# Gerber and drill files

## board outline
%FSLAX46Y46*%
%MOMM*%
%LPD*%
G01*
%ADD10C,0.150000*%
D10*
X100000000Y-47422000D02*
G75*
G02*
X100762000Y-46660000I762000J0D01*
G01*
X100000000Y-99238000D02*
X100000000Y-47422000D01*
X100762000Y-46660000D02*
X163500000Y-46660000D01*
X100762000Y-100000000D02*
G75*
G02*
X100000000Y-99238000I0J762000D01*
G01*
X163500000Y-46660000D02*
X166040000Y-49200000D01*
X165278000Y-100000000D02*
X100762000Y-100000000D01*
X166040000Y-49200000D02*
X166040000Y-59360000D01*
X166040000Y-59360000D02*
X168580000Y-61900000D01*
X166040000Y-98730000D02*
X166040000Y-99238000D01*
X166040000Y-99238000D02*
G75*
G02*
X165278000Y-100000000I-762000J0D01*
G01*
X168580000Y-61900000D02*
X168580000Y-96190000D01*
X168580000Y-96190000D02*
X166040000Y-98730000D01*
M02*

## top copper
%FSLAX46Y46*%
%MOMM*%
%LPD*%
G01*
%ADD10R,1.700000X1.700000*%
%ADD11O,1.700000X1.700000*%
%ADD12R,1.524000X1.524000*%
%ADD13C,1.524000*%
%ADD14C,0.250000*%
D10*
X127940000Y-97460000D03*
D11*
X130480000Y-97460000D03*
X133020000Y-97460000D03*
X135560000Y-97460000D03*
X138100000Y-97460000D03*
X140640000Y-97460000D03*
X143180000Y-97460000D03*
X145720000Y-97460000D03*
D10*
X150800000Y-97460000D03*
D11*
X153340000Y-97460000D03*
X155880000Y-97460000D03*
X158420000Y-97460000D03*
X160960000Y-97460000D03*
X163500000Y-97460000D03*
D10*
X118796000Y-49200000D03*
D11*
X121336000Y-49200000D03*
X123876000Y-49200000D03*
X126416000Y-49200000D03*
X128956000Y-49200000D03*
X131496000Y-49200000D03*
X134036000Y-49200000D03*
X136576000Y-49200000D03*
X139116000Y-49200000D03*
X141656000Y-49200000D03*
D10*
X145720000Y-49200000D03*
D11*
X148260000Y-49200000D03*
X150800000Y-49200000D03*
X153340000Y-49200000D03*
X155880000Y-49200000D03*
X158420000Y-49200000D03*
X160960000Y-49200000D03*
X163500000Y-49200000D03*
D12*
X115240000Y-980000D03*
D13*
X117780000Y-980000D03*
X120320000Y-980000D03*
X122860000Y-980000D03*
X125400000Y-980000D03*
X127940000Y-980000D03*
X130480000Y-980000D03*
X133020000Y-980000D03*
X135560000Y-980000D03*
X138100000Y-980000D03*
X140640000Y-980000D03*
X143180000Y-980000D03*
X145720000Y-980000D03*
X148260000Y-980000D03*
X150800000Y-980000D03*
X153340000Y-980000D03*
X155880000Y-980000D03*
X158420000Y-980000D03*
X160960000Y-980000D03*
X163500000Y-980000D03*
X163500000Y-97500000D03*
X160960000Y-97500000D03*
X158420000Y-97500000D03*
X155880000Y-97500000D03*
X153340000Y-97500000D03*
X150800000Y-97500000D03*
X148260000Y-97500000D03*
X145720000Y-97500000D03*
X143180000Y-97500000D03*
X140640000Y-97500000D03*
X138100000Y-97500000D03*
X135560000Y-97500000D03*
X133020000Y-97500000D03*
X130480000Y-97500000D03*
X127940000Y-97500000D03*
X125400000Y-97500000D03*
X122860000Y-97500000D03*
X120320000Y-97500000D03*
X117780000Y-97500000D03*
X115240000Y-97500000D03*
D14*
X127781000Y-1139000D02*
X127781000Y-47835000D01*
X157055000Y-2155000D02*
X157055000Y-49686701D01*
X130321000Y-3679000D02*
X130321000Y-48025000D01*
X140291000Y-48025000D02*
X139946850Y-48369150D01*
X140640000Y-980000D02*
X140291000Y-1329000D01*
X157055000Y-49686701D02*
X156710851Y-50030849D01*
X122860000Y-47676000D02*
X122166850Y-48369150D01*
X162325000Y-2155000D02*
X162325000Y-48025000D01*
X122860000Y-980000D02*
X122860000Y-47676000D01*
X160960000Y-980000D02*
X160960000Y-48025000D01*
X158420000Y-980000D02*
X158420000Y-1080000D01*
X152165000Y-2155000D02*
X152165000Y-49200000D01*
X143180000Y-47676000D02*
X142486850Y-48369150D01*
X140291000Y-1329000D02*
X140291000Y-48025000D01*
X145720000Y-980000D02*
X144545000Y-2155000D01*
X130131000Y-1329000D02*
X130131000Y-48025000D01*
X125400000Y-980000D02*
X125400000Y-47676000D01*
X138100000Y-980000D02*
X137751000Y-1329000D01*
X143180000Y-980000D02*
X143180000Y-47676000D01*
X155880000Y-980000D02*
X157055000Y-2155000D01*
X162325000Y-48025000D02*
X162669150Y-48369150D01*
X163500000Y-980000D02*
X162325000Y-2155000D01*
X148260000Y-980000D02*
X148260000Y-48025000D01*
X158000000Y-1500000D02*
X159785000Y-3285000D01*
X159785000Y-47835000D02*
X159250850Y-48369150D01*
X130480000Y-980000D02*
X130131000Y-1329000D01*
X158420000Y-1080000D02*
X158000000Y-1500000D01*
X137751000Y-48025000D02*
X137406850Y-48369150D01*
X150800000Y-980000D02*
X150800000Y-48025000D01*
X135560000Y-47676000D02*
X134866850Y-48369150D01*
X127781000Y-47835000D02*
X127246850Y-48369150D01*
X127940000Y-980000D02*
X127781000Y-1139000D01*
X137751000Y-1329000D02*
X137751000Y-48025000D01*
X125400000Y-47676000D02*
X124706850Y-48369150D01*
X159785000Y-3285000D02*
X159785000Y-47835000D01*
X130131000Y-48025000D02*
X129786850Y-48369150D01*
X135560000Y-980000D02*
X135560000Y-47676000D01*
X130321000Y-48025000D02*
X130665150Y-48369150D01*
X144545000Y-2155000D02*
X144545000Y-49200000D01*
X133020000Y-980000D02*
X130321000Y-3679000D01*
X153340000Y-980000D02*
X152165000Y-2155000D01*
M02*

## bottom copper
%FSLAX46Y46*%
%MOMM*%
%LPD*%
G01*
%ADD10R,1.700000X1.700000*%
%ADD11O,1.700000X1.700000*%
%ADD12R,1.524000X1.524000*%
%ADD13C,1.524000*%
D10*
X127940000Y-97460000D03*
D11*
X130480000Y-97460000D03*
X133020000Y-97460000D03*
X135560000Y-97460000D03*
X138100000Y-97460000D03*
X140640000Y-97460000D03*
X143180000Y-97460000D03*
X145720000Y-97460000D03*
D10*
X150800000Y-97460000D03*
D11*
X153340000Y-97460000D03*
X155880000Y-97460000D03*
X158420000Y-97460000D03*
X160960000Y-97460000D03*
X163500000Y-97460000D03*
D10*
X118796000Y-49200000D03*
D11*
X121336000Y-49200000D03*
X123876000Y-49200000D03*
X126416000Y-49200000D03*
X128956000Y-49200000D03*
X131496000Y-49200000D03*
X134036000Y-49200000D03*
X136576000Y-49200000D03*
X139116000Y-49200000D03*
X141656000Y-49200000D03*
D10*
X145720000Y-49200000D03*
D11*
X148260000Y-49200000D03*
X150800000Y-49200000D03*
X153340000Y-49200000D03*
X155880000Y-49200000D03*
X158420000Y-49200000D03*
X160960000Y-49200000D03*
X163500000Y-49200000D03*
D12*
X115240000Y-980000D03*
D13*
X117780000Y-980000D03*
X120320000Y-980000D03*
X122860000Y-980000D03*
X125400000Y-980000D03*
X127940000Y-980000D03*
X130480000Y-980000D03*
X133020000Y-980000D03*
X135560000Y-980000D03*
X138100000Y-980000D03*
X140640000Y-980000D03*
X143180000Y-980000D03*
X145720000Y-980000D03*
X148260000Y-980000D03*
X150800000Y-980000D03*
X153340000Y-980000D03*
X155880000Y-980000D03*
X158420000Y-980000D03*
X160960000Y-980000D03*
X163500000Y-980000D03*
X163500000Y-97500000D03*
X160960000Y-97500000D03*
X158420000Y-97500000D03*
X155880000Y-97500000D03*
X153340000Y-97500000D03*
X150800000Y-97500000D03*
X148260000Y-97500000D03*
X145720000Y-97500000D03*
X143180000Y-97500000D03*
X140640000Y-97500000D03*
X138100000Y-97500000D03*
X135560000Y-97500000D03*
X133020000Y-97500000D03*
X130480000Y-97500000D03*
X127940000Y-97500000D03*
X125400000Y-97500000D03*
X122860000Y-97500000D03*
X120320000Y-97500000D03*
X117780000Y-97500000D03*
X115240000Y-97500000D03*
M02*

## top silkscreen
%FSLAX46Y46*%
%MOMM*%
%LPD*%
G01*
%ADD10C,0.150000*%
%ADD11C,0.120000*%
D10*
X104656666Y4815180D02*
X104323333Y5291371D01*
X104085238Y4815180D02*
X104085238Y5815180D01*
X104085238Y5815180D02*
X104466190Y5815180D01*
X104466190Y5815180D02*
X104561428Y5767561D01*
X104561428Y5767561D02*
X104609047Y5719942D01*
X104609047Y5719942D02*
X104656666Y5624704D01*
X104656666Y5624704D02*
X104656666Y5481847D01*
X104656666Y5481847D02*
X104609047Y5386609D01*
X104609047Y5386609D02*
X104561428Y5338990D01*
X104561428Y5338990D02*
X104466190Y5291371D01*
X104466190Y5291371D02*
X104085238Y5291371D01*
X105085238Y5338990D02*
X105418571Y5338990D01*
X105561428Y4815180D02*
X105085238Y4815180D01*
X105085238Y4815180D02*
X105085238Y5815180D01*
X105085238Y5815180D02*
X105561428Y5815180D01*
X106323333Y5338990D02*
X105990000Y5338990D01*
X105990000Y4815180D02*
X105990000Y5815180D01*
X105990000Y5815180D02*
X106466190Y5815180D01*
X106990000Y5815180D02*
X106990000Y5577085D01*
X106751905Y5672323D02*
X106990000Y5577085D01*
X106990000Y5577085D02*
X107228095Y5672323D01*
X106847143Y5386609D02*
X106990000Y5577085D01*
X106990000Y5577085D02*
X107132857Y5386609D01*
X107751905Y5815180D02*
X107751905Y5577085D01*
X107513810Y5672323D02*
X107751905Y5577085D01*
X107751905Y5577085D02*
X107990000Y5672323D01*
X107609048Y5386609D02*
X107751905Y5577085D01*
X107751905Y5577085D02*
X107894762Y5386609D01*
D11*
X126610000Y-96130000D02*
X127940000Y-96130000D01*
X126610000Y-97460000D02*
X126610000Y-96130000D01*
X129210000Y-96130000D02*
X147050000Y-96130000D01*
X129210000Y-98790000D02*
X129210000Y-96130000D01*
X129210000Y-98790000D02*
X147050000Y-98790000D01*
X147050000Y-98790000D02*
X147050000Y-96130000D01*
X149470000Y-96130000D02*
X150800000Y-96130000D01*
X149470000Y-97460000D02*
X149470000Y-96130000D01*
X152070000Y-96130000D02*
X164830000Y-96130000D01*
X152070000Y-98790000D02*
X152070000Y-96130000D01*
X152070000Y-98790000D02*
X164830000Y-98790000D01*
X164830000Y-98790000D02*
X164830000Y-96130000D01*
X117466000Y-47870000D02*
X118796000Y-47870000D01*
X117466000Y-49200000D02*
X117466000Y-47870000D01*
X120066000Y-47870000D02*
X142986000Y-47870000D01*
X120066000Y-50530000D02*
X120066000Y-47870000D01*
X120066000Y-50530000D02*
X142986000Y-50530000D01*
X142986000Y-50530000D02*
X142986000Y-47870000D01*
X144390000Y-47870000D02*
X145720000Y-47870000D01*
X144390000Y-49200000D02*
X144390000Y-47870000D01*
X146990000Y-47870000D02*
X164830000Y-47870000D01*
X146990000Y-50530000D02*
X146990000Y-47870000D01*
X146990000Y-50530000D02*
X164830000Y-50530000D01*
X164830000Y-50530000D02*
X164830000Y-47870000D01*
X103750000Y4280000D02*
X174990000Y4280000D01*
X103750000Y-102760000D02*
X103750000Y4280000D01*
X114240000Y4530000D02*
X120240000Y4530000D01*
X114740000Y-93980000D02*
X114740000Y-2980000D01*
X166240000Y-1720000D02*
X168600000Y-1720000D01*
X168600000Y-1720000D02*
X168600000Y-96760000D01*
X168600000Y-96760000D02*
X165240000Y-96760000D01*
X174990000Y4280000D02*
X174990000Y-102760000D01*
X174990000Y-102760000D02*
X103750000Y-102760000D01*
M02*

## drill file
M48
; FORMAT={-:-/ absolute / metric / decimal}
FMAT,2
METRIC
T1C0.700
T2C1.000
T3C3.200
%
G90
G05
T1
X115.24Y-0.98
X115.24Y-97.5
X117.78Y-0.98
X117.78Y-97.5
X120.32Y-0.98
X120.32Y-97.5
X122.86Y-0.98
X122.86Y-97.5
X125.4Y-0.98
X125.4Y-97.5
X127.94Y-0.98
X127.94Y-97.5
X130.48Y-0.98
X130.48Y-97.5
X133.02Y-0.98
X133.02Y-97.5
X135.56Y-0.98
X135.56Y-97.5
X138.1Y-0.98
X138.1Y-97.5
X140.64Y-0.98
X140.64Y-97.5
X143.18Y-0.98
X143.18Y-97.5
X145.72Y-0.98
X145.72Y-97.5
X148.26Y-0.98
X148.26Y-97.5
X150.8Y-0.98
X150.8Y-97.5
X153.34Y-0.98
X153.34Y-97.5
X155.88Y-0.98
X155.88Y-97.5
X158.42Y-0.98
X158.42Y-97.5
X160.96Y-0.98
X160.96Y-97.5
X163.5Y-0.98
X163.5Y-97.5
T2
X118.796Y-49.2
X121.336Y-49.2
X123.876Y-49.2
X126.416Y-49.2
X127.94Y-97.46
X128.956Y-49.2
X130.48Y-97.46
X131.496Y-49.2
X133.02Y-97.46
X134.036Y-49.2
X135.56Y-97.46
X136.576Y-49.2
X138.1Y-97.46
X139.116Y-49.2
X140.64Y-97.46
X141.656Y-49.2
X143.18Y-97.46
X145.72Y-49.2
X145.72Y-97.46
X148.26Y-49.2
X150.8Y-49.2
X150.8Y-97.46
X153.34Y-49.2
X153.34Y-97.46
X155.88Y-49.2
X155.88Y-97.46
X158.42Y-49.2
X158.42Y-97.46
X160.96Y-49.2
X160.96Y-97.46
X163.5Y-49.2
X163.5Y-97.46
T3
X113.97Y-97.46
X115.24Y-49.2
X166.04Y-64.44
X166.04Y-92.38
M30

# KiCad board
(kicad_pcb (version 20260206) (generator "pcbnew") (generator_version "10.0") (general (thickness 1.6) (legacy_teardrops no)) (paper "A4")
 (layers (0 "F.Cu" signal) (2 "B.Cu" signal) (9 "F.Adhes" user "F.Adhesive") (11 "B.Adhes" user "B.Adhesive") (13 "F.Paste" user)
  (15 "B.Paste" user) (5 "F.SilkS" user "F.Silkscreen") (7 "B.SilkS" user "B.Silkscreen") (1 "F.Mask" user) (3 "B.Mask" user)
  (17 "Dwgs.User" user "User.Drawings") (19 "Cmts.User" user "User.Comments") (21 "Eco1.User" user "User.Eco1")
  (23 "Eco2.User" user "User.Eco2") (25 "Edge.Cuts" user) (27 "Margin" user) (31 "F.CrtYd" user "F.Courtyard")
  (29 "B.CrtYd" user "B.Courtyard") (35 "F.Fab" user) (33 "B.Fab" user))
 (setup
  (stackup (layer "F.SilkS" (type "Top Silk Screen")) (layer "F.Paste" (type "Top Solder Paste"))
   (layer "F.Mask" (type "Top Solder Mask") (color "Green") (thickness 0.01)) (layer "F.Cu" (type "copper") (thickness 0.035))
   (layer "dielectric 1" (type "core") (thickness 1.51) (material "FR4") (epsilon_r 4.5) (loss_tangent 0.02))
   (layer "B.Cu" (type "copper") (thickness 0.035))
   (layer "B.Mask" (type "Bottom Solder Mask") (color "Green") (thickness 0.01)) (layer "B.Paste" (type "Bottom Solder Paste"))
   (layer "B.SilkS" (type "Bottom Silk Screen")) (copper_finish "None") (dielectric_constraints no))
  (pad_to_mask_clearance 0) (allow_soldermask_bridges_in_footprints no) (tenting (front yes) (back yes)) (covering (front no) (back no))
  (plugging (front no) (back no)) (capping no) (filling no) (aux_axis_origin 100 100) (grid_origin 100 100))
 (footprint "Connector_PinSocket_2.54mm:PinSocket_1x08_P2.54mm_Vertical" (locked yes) (layer "F.Cu") (at 127.94 97.46 90)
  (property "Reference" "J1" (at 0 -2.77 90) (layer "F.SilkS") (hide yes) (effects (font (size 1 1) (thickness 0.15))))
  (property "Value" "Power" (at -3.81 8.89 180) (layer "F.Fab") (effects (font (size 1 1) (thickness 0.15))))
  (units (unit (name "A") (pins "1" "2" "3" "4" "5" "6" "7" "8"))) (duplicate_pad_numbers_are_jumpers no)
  (fp_line (start 1.33 -1.33) (end 1.33 0) (stroke (width 0.12) (type solid)) (layer "F.SilkS"))
  (fp_line (start 0 -1.33) (end 1.33 -1.33) (stroke (width 0.12) (type solid)) (layer "F.SilkS"))
  (fp_line (start 1.33 1.27) (end 1.33 19.11) (stroke (width 0.12) (type solid)) (layer "F.SilkS"))
  (fp_line (start -1.33 1.27) (end 1.33 1.27) (stroke (width 0.12) (type solid)) (layer "F.SilkS"))
  (fp_line (start -1.33 1.27) (end -1.33 19.11) (stroke (width 0.12) (type solid)) (layer "F.SilkS"))
  (fp_line (start -1.33 19.11) (end 1.33 19.11) (stroke (width 0.12) (type solid)) (layer "F.SilkS"))
  (pad "1" thru_hole rect (at 0 0 90) (size 1.7 1.7) (drill 1) (layers "*.Cu" "*.Mask") (remove_unused_layers no)
   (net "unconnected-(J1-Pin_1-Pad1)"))
  (pad "2" thru_hole oval (at 0 2.54 90) (size 1.7 1.7) (drill 1) (layers "*.Cu" "*.Mask") (remove_unused_layers no) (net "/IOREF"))
  (pad "3" thru_hole oval (at 0 5.08 90) (size 1.7 1.7) (drill 1) (layers "*.Cu" "*.Mask") (remove_unused_layers no) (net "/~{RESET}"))
  (pad "4" thru_hole oval (at 0 7.62 90) (size 1.7 1.7) (drill 1) (layers "*.Cu" "*.Mask") (remove_unused_layers no) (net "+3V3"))
  (pad "5" thru_hole oval (at 0 10.16 90) (size 1.7 1.7) (drill 1) (layers "*.Cu" "*.Mask") (remove_unused_layers no) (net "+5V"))
  (pad "6" thru_hole oval (at 0 12.7 90) (size 1.7 1.7) (drill 1) (layers "*.Cu" "*.Mask") (remove_unused_layers no) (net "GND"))
  (pad "7" thru_hole oval (at 0 15.24 90) (size 1.7 1.7) (drill 1) (layers "*.Cu" "*.Mask") (remove_unused_layers no) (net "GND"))
  (pad "8" thru_hole oval (at 0 17.78 90) (size 1.7 1.7) (drill 1) (layers "*.Cu" "*.Mask") (remove_unused_layers no) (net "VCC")))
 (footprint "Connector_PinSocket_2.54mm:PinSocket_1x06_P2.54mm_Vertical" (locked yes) (layer "F.Cu") (at 150.8 97.46 90)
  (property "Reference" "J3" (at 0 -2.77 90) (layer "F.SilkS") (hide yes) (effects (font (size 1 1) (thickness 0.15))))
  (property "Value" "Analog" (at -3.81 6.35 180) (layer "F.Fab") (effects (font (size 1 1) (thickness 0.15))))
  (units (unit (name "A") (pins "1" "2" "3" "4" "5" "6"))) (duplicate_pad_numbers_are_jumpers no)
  (fp_line (start 1.33 -1.33) (end 1.33 0) (stroke (width 0.12) (type solid)) (layer "F.SilkS"))
  (fp_line (start 0 -1.33) (end 1.33 -1.33) (stroke (width 0.12) (type solid)) (layer "F.SilkS"))
  (fp_line (start 1.33 1.27) (end 1.33 14.03) (stroke (width 0.12) (type solid)) (layer "F.SilkS"))
  (fp_line (start -1.33 1.27) (end 1.33 1.27) (stroke (width 0.12) (type solid)) (layer "F.SilkS"))
  (fp_line (start -1.33 1.27) (end -1.33 14.03) (stroke (width 0.12) (type solid)) (layer "F.SilkS"))
  (fp_line (start -1.33 14.03) (end 1.33 14.03) (stroke (width 0.12) (type solid)) (layer "F.SilkS"))
  (pad "1" thru_hole rect (at 0 0 90) (size 1.7 1.7) (drill 1) (layers "*.Cu" "*.Mask") (remove_unused_layers no) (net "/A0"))
  (pad "2" thru_hole oval (at 0 2.54 90) (size 1.7 1.7) (drill 1) (layers "*.Cu" "*.Mask") (remove_unused_layers no) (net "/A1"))
  (pad "3" thru_hole oval (at 0 5.08 90) (size 1.7 1.7) (drill 1) (layers "*.Cu" "*.Mask") (remove_unused_layers no) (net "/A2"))
  (pad "4" thru_hole oval (at 0 7.62 90) (size 1.7 1.7) (drill 1) (layers "*.Cu" "*.Mask") (remove_unused_layers no) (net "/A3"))
  (pad "5" thru_hole oval (at 0 10.16 90) (size 1.7 1.7) (drill 1) (layers "*.Cu" "*.Mask") (remove_unused_layers no) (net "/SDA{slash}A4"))
  (pad "6" thru_hole oval (at 0 12.7 90) (size 1.7 1.7) (drill 1) (layers "*.Cu" "*.Mask") (remove_unused_layers no) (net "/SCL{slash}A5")))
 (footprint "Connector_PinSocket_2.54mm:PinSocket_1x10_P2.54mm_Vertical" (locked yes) (layer "F.Cu") (at 118.796 49.2 90)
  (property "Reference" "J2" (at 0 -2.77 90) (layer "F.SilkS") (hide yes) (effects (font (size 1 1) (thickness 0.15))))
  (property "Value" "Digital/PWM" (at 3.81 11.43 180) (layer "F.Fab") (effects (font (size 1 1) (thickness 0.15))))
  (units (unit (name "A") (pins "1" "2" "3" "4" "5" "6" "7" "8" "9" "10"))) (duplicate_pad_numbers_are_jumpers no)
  (fp_line (start 1.33 -1.33) (end 1.33 0) (stroke (width 0.12) (type solid)) (layer "F.SilkS"))
  (fp_line (start 0 -1.33) (end 1.33 -1.33) (stroke (width 0.12) (type solid)) (layer "F.SilkS"))
  (fp_line (start 1.33 1.27) (end 1.33 24.19) (stroke (width 0.12) (type solid)) (layer "F.SilkS"))
  (fp_line (start -1.33 1.27) (end 1.33 1.27) (stroke (width 0.12) (type solid)) (layer "F.SilkS"))
  (fp_line (start -1.33 1.27) (end -1.33 24.19) (stroke (width 0.12) (type solid)) (layer "F.SilkS"))
  (fp_line (start -1.33 24.19) (end 1.33 24.19) (stroke (width 0.12) (type solid)) (layer "F.SilkS"))
  (pad "1" thru_hole rect (at 0 0 90) (size 1.7 1.7) (drill 1) (layers "*.Cu" "*.Mask") (remove_unused_layers no) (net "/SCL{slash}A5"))
  (pad "2" thru_hole oval (at 0 2.54 90) (size 1.7 1.7) (drill 1) (layers "*.Cu" "*.Mask") (remove_unused_layers no) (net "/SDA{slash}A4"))
  (pad "3" thru_hole oval (at 0 5.08 90) (size 1.7 1.7) (drill 1) (layers "*.Cu" "*.Mask") (remove_unused_layers no) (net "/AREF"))
  (pad "4" thru_hole oval (at 0 7.62 90) (size 1.7 1.7) (drill 1) (layers "*.Cu" "*.Mask") (remove_unused_layers no) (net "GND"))
  (pad "5" thru_hole oval (at 0 10.16 90) (size 1.7 1.7) (drill 1) (layers "*.Cu" "*.Mask") (remove_unused_layers no) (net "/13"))
  (pad "6" thru_hole oval (at 0 12.7 90) (size 1.7 1.7) (drill 1) (layers "*.Cu" "*.Mask") (remove_unused_layers no) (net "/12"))
  (pad "7" thru_hole oval (at 0 15.24 90) (size 1.7 1.7) (drill 1) (layers "*.Cu" "*.Mask") (remove_unused_layers no) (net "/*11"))
  (pad "8" thru_hole oval (at 0 17.78 90) (size 1.7 1.7) (drill 1) (layers "*.Cu" "*.Mask") (remove_unused_layers no) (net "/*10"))
  (pad "9" thru_hole oval (at 0 20.32 90) (size 1.7 1.7) (drill 1) (layers "*.Cu" "*.Mask") (remove_unused_layers no) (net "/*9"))
  (pad "10" thru_hole oval (at 0 22.86 90) (size 1.7 1.7) (drill 1) (layers "*.Cu" "*.Mask") (remove_unused_layers no) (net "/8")))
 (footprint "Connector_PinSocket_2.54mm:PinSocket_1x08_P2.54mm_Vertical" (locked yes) (layer "F.Cu") (at 145.72 49.2 90)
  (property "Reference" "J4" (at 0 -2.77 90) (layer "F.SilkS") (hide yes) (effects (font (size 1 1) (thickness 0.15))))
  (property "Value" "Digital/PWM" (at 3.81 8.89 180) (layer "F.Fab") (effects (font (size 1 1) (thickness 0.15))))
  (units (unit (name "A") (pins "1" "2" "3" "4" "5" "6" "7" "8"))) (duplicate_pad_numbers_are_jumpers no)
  (fp_line (start 1.33 -1.33) (end 1.33 0) (stroke (width 0.12) (type solid)) (layer "F.SilkS"))
  (fp_line (start 0 -1.33) (end 1.33 -1.33) (stroke (width 0.12) (type solid)) (layer "F.SilkS"))
  (fp_line (start 1.33 1.27) (end 1.33 19.11) (stroke (width 0.12) (type solid)) (layer "F.SilkS"))
  (fp_line (start -1.33 1.27) (end 1.33 1.27) (stroke (width 0.12) (type solid)) (layer "F.SilkS"))
  (fp_line (start -1.33 1.27) (end -1.33 19.11) (stroke (width 0.12) (type solid)) (layer "F.SilkS"))
  (fp_line (start -1.33 19.11) (end 1.33 19.11) (stroke (width 0.12) (type solid)) (layer "F.SilkS"))
  (pad "1" thru_hole rect (at 0 0 90) (size 1.7 1.7) (drill 1) (layers "*.Cu" "*.Mask") (remove_unused_layers no) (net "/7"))
  (pad "2" thru_hole oval (at 0 2.54 90) (size 1.7 1.7) (drill 1) (layers "*.Cu" "*.Mask") (remove_unused_layers no) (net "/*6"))
  (pad "3" thru_hole oval (at 0 5.08 90) (size 1.7 1.7) (drill 1) (layers "*.Cu" "*.Mask") (remove_unused_layers no) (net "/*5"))
  (pad "4" thru_hole oval (at 0 7.62 90) (size 1.7 1.7) (drill 1) (layers "*.Cu" "*.Mask") (remove_unused_layers no) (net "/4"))
  (pad "5" thru_hole oval (at 0 10.16 90) (size 1.7 1.7) (drill 1) (layers "*.Cu" "*.Mask") (remove_unused_layers no) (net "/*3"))
  (pad "6" thru_hole oval (at 0 12.7 90) (size 1.7 1.7) (drill 1) (layers "*.Cu" "*.Mask") (remove_unused_layers no) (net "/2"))
  (pad "7" thru_hole oval (at 0 15.24 90) (size 1.7 1.7) (drill 1) (layers "*.Cu" "*.Mask") (remove_unused_layers no) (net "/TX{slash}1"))
  (pad "8" thru_hole oval (at 0 17.78 90) (size 1.7 1.7) (drill 1) (layers "*.Cu" "*.Mask") (remove_unused_layers no) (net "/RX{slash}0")))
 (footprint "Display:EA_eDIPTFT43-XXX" (layer "F.Cu") (at 115.24 0.98)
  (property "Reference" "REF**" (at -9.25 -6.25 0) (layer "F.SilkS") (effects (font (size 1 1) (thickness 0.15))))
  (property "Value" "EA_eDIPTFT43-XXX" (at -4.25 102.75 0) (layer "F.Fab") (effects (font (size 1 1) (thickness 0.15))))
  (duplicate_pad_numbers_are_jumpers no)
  (fp_line (start -11.49 -5.26) (end 59.75 -5.26) (stroke (width 0.12) (type solid)) (layer "F.SilkS"))
  (fp_line (start -11.49 101.78) (end -11.49 -5.26) (stroke (width 0.12) (type solid)) (layer "F.SilkS"))
  (fp_line (start -1 -5.51) (end 5 -5.51) (stroke (width 0.12) (type solid)) (layer "F.SilkS"))
  (fp_line (start -0.5 93) (end -0.5 2) (stroke (width 0.12) (type solid)) (layer "F.SilkS"))
  (fp_line (start 51 0.74) (end 53.36 0.74) (stroke (width 0.12) (type solid)) (layer "F.SilkS"))
  (fp_line (start 53.36 0.74) (end 53.36 95.78) (stroke (width 0.12) (type solid)) (layer "F.SilkS"))
  (fp_line (start 53.36 95.78) (end 50 95.78) (stroke (width 0.12) (type solid)) (layer "F.SilkS"))
  (fp_line (start 59.75 -5.26) (end 59.75 101.78) (stroke (width 0.12) (type solid)) (layer "F.SilkS"))
  (fp_line (start 59.75 101.78) (end -11.49 101.78) (stroke (width 0.12) (type solid)) (layer "F.SilkS"))
  (pad "1" thru_hole rect (at 0 0) (size 1.524 1.524) (drill 0.7) (layers "*.Cu" "*.Mask") (remove_unused_layers no))
  (pad "2" thru_hole circle (at 2.54 0) (size 1.524 1.524) (drill 0.7) (layers "*.Cu" "*.Mask") (remove_unused_layers no))
  (pad "3" thru_hole circle (at 5.08 0) (size 1.524 1.524) (drill 0.7) (layers "*.Cu" "*.Mask") (remove_unused_layers no))
  (pad "4" thru_hole circle (at 7.62 0) (size 1.524 1.524) (drill 0.7) (layers "*.Cu" "*.Mask") (remove_unused_layers no))
  (pad "5" thru_hole circle (at 10.16 0) (size 1.524 1.524) (drill 0.7) (layers "*.Cu" "*.Mask") (remove_unused_layers no))
  (pad "6" thru_hole circle (at 12.7 0) (size 1.524 1.524) (drill 0.7) (layers "*.Cu" "*.Mask") (remove_unused_layers no))
  (pad "7" thru_hole circle (at 15.24 0) (size 1.524 1.524) (drill 0.7) (layers "*.Cu" "*.Mask") (remove_unused_layers no))
  (pad "8" thru_hole circle (at 17.78 0) (size 1.524 1.524) (drill 0.7) (layers "*.Cu" "*.Mask") (remove_unused_layers no))
  (pad "9" thru_hole circle (at 20.32 0) (size 1.524 1.524) (drill 0.7) (layers "*.Cu" "*.Mask") (remove_unused_layers no))
  (pad "10" thru_hole circle (at 22.86 0) (size 1.524 1.524) (drill 0.7) (layers "*.Cu" "*.Mask") (remove_unused_layers no))
  (pad "11" thru_hole circle (at 25.4 0) (size 1.524 1.524) (drill 0.7) (layers "*.Cu" "*.Mask") (remove_unused_layers no))
  (pad "12" thru_hole circle (at 27.94 0) (size 1.524 1.524) (drill 0.7) (layers "*.Cu" "*.Mask") (remove_unused_layers no))
  (pad "13" thru_hole circle (at 30.48 0) (size 1.524 1.524) (drill 0.7) (layers "*.Cu" "*.Mask") (remove_unused_layers no))
  (pad "14" thru_hole circle (at 33.02 0) (size 1.524 1.524) (drill 0.7) (layers "*.Cu" "*.Mask") (remove_unused_layers no))
  (pad "15" thru_hole circle (at 35.56 0) (size 1.524 1.524) (drill 0.7) (layers "*.Cu" "*.Mask") (remove_unused_layers no))
  (pad "16" thru_hole circle (at 38.1 0) (size 1.524 1.524) (drill 0.7) (layers "*.Cu" "*.Mask") (remove_unused_layers no))
  (pad "17" thru_hole circle (at 40.64 0) (size 1.524 1.524) (drill 0.7) (layers "*.Cu" "*.Mask") (remove_unused_layers no))
  (pad "18" thru_hole circle (at 43.18 0) (size 1.524 1.524) (drill 0.7) (layers "*.Cu" "*.Mask") (remove_unused_layers no))
  (pad "19" thru_hole circle (at 45.72 0) (size 1.524 1.524) (drill 0.7) (layers "*.Cu" "*.Mask") (remove_unused_layers no))
  (pad "20" thru_hole circle (at 48.26 0) (size 1.524 1.524) (drill 0.7) (layers "*.Cu" "*.Mask") (remove_unused_layers no))
  (pad "21" thru_hole circle (at 48.26 96.52) (size 1.524 1.524) (drill 0.7) (layers "*.Cu" "*.Mask") (remove_unused_layers no))
  (pad "22" thru_hole circle (at 45.72 96.52) (size 1.524 1.524) (drill 0.7) (layers "*.Cu" "*.Mask") (remove_unused_layers no))
  (pad "23" thru_hole circle (at 43.18 96.52) (size 1.524 1.524) (drill 0.7) (layers "*.Cu" "*.Mask") (remove_unused_layers no))
  (pad "24" thru_hole circle (at 40.64 96.52) (size 1.524 1.524) (drill 0.7) (layers "*.Cu" "*.Mask") (remove_unused_layers no))
  (pad "25" thru_hole circle (at 38.1 96.52) (size 1.524 1.524) (drill 0.7) (layers "*.Cu" "*.Mask") (remove_unused_layers no))
  (pad "26" thru_hole circle (at 35.56 96.52) (size 1.524 1.524) (drill 0.7) (layers "*.Cu" "*.Mask") (remove_unused_layers no))
  (pad "27" thru_hole circle (at 33.02 96.52) (size 1.524 1.524) (drill 0.7) (layers "*.Cu" "*.Mask") (remove_unused_layers no))
  (pad "28" thru_hole circle (at 30.48 96.52) (size 1.524 1.524) (drill 0.7) (layers "*.Cu" "*.Mask") (remove_unused_layers no))
  (pad "29" thru_hole circle (at 27.94 96.52) (size 1.524 1.524) (drill 0.7) (layers "*.Cu" "*.Mask") (remove_unused_layers no))
  (pad "30" thru_hole circle (at 25.4 96.52) (size 1.524 1.524) (drill 0.7) (layers "*.Cu" "*.Mask") (remove_unused_layers no))
  (pad "31" thru_hole circle (at 22.86 96.52) (size 1.524 1.524) (drill 0.7) (layers "*.Cu" "*.Mask") (remove_unused_layers no))
  (pad "32" thru_hole circle (at 20.32 96.52) (size 1.524 1.524) (drill 0.7) (layers "*.Cu" "*.Mask") (remove_unused_layers no))
  (pad "33" thru_hole circle (at 17.78 96.52) (size 1.524 1.524) (drill 0.7) (layers "*.Cu" "*.Mask") (remove_unused_layers no))
  (pad "34" thru_hole circle (at 15.24 96.52) (size 1.524 1.524) (drill 0.7) (layers "*.Cu" "*.Mask") (remove_unused_layers no))
  (pad "35" thru_hole circle (at 12.7 96.52) (size 1.524 1.524) (drill 0.7) (layers "*.Cu" "*.Mask") (remove_unused_layers no))
  (pad "36" thru_hole circle (at 10.16 96.52) (size 1.524 1.524) (drill 0.7) (layers "*.Cu" "*.Mask") (remove_unused_layers no))
  (pad "37" thru_hole circle (at 7.62 96.52) (size 1.524 1.524) (drill 0.7) (layers "*.Cu" "*.Mask") (remove_unused_layers no))
  (pad "38" thru_hole circle (at 5.08 96.52) (size 1.524 1.524) (drill 0.7) (layers "*.Cu" "*.Mask") (remove_unused_layers no))
  (pad "39" thru_hole circle (at 2.54 96.52) (size 1.524 1.524) (drill 0.7) (layers "*.Cu" "*.Mask") (remove_unused_layers no))
  (pad "40" thru_hole circle (at 0 96.52) (size 1.524 1.524) (drill 0.7) (layers "*.Cu" "*.Mask") (remove_unused_layers no)))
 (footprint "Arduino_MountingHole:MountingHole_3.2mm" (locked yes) (layer "F.Cu") (at 115.24 49.2)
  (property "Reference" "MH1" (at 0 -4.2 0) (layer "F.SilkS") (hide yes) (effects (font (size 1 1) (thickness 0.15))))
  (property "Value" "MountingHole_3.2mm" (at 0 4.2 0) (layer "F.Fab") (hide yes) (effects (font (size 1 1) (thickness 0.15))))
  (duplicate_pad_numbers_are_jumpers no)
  (pad "" np_thru_hole circle (at 0 0) (size 3.2 3.2) (drill 3.2) (layers "*.Cu" "*.Mask")))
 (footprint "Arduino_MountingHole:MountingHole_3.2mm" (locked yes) (layer "F.Cu") (at 113.97 97.46)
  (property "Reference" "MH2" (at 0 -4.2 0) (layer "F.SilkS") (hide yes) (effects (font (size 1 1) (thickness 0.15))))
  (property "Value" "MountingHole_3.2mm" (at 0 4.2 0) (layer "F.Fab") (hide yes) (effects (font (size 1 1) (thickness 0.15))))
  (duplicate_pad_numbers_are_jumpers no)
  (pad "" np_thru_hole circle (at 0 0) (size 3.2 3.2) (drill 3.2) (layers "*.Cu" "*.Mask")))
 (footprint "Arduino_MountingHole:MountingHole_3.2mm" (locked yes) (layer "F.Cu") (at 166.04 64.44)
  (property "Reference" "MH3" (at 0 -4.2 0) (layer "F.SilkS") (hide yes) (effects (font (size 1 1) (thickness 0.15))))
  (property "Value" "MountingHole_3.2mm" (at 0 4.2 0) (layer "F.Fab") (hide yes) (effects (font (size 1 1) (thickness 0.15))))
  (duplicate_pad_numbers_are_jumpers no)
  (pad "" np_thru_hole circle (at 0 0) (size 3.2 3.2) (drill 3.2) (layers "*.Cu" "*.Mask")))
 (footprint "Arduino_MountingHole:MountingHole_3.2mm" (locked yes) (layer "F.Cu") (at 166.04 92.38)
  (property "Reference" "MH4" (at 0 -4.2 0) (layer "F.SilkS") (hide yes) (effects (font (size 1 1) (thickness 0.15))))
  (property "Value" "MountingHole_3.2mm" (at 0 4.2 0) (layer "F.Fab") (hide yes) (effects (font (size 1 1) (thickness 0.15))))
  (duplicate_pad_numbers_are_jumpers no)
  (pad "" np_thru_hole circle (at 0 0) (size 3.2 3.2) (drill 3.2) (layers "*.Cu" "*.Mask")))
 (gr_arc (start 100 47.422) (mid 100.223185 46.883185) (end 100.762 46.66) (stroke (width 0.15) (type solid)) (layer "Edge.Cuts"))
 (gr_line (start 100 99.238) (end 100 47.422) (stroke (width 0.15) (type solid)) (layer "Edge.Cuts"))
 (gr_line (start 100.762 46.66) (end 163.5 46.66) (stroke (width 0.15) (type solid)) (layer "Edge.Cuts"))
 (gr_arc (start 100.762 100) (mid 100.223185 99.776815) (end 100 99.238) (stroke (width 0.15) (type solid)) (layer "Edge.Cuts"))
 (gr_line (start 163.5 46.66) (end 166.04 49.2) (stroke (width 0.15) (type solid)) (layer "Edge.Cuts"))
 (gr_line (start 165.278 100) (end 100.762 100) (stroke (width 0.15) (type solid)) (layer "Edge.Cuts"))
 (gr_line (start 166.04 49.2) (end 166.04 59.36) (stroke (width 0.15) (type solid)) (layer "Edge.Cuts"))
 (gr_line (start 166.04 59.36) (end 168.58 61.9) (stroke (width 0.15) (type solid)) (layer "Edge.Cuts"))
 (gr_line (start 166.04 98.73) (end 166.04 99.238) (stroke (width 0.15) (type solid)) (layer "Edge.Cuts"))
 (gr_arc (start 166.04 99.238) (mid 165.816815 99.776815) (end 165.278 100) (stroke (width 0.15) (type solid)) (layer "Edge.Cuts"))
 (gr_line (start 168.58 61.9) (end 168.58 96.19) (stroke (width 0.15) (type solid)) (layer "Edge.Cuts"))
 (gr_line (start 168.58 96.19) (end 166.04 98.73) (stroke (width 0.15) (type solid)) (layer "Edge.Cuts"))
 (segment (start 127.781 1.139) (end 127.781 47.835) (width 0.25) (layer "F.Cu") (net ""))
 (segment (start 157.055 2.155) (end 157.055 49.686701) (width 0.25) (layer "F.Cu") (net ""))
 (segment (start 130.321 3.679) (end 130.321 48.025) (width 0.25) (layer "F.Cu") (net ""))
 (segment (start 140.291 48.025) (end 139.94685 48.36915) (width 0.25) (layer "F.Cu") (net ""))
 (segment (start 140.64 0.98) (end 140.291 1.329) (width 0.25) (layer "F.Cu") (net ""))
 (segment (start 157.055 49.686701) (end 156.710851 50.030849) (width 0.25) (layer "F.Cu") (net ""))
 (segment (start 122.86 47.676) (end 122.16685 48.36915) (width 0.25) (layer "F.Cu") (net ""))
 (segment (start 162.325 2.155) (end 162.325 48.025) (width 0.25) (layer "F.Cu") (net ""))
 (segment (start 122.86 0.98) (end 122.86 47.676) (width 0.25) (layer "F.Cu") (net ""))
 (segment (start 160.96 0.98) (end 160.96 48.025) (width 0.25) (layer "F.Cu") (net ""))
 (segment (start 158.42 0.98) (end 158.42 1.08) (width 0.25) (layer "F.Cu") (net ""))
 (segment (start 152.165 2.155) (end 152.165 49.2) (width 0.25) (layer "F.Cu") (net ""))
 (segment (start 143.18 47.676) (end 142.48685 48.36915) (width 0.25) (layer "F.Cu") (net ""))
 (segment (start 140.291 1.329) (end 140.291 48.025) (width 0.25) (layer "F.Cu") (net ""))
 (segment (start 145.72 0.98) (end 144.545 2.155) (width 0.25) (layer "F.Cu") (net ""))
 (segment (start 130.131 1.329) (end 130.131 48.025) (width 0.25) (layer "F.Cu") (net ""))
 (segment (start 125.4 0.98) (end 125.4 47.676) (width 0.25) (layer "F.Cu") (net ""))
 (segment (start 138.1 0.98) (end 137.751 1.329) (width 0.25) (layer "F.Cu") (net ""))
 (segment (start 143.18 0.98) (end 143.18 47.676) (width 0.25) (layer "F.Cu") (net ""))
 (segment (start 155.88 0.98) (end 157.055 2.155) (width 0.25) (layer "F.Cu") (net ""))
 (segment (start 162.325 48.025) (end 162.66915 48.36915) (width 0.25) (layer "F.Cu") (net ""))
 (segment (start 163.5 0.98) (end 162.325 2.155) (width 0.25) (layer "F.Cu") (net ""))
 (segment (start 148.26 0.98) (end 148.26 48.025) (width 0.25) (layer "F.Cu") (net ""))
 (segment (start 158 1.5) (end 159.785 3.285) (width 0.25) (layer "F.Cu") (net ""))
 (segment (start 159.785 47.835) (end 159.25085 48.36915) (width 0.25) (layer "F.Cu") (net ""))
 (segment (start 130.48 0.98) (end 130.131 1.329) (width 0.25) (layer "F.Cu") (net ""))
 (segment (start 158.42 1.08) (end 158 1.5) (width 0.25) (layer "F.Cu") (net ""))
 (segment (start 137.751 48.025) (end 137.40685 48.36915) (width 0.25) (layer "F.Cu") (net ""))
 (segment (start 150.8 0.98) (end 150.8 48.025) (width 0.25) (layer "F.Cu") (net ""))
 (segment (start 135.56 47.676) (end 134.86685 48.36915) (width 0.25) (layer "F.Cu") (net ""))
 (segment (start 127.781 47.835) (end 127.24685 48.36915) (width 0.25) (layer "F.Cu") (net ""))
 (segment (start 127.94 0.98) (end 127.781 1.139) (width 0.25) (layer "F.Cu") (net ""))
 (segment (start 137.751 1.329) (end 137.751 48.025) (width 0.25) (layer "F.Cu") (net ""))
 (segment (start 125.4 47.676) (end 124.70685 48.36915) (width 0.25) (layer "F.Cu") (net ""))
 (segment (start 159.785 3.285) (end 159.785 47.835) (width 0.25) (layer "F.Cu") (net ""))
 (segment (start 130.131 48.025) (end 129.78685 48.36915) (width 0.25) (layer "F.Cu") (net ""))
 (segment (start 135.56 0.98) (end 135.56 47.676) (width 0.25) (layer "F.Cu") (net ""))
 (segment (start 130.321 48.025) (end 130.66515 48.36915) (width 0.25) (layer "F.Cu") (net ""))
 (segment (start 144.545 2.155) (end 144.545 49.2) (width 0.25) (layer "F.Cu") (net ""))
 (segment (start 133.02 0.98) (end 130.321 3.679) (width 0.25) (layer "F.Cu") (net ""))
 (segment (start 153.34 0.98) (end 152.165 2.155) (width 0.25) (layer "F.Cu") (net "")))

